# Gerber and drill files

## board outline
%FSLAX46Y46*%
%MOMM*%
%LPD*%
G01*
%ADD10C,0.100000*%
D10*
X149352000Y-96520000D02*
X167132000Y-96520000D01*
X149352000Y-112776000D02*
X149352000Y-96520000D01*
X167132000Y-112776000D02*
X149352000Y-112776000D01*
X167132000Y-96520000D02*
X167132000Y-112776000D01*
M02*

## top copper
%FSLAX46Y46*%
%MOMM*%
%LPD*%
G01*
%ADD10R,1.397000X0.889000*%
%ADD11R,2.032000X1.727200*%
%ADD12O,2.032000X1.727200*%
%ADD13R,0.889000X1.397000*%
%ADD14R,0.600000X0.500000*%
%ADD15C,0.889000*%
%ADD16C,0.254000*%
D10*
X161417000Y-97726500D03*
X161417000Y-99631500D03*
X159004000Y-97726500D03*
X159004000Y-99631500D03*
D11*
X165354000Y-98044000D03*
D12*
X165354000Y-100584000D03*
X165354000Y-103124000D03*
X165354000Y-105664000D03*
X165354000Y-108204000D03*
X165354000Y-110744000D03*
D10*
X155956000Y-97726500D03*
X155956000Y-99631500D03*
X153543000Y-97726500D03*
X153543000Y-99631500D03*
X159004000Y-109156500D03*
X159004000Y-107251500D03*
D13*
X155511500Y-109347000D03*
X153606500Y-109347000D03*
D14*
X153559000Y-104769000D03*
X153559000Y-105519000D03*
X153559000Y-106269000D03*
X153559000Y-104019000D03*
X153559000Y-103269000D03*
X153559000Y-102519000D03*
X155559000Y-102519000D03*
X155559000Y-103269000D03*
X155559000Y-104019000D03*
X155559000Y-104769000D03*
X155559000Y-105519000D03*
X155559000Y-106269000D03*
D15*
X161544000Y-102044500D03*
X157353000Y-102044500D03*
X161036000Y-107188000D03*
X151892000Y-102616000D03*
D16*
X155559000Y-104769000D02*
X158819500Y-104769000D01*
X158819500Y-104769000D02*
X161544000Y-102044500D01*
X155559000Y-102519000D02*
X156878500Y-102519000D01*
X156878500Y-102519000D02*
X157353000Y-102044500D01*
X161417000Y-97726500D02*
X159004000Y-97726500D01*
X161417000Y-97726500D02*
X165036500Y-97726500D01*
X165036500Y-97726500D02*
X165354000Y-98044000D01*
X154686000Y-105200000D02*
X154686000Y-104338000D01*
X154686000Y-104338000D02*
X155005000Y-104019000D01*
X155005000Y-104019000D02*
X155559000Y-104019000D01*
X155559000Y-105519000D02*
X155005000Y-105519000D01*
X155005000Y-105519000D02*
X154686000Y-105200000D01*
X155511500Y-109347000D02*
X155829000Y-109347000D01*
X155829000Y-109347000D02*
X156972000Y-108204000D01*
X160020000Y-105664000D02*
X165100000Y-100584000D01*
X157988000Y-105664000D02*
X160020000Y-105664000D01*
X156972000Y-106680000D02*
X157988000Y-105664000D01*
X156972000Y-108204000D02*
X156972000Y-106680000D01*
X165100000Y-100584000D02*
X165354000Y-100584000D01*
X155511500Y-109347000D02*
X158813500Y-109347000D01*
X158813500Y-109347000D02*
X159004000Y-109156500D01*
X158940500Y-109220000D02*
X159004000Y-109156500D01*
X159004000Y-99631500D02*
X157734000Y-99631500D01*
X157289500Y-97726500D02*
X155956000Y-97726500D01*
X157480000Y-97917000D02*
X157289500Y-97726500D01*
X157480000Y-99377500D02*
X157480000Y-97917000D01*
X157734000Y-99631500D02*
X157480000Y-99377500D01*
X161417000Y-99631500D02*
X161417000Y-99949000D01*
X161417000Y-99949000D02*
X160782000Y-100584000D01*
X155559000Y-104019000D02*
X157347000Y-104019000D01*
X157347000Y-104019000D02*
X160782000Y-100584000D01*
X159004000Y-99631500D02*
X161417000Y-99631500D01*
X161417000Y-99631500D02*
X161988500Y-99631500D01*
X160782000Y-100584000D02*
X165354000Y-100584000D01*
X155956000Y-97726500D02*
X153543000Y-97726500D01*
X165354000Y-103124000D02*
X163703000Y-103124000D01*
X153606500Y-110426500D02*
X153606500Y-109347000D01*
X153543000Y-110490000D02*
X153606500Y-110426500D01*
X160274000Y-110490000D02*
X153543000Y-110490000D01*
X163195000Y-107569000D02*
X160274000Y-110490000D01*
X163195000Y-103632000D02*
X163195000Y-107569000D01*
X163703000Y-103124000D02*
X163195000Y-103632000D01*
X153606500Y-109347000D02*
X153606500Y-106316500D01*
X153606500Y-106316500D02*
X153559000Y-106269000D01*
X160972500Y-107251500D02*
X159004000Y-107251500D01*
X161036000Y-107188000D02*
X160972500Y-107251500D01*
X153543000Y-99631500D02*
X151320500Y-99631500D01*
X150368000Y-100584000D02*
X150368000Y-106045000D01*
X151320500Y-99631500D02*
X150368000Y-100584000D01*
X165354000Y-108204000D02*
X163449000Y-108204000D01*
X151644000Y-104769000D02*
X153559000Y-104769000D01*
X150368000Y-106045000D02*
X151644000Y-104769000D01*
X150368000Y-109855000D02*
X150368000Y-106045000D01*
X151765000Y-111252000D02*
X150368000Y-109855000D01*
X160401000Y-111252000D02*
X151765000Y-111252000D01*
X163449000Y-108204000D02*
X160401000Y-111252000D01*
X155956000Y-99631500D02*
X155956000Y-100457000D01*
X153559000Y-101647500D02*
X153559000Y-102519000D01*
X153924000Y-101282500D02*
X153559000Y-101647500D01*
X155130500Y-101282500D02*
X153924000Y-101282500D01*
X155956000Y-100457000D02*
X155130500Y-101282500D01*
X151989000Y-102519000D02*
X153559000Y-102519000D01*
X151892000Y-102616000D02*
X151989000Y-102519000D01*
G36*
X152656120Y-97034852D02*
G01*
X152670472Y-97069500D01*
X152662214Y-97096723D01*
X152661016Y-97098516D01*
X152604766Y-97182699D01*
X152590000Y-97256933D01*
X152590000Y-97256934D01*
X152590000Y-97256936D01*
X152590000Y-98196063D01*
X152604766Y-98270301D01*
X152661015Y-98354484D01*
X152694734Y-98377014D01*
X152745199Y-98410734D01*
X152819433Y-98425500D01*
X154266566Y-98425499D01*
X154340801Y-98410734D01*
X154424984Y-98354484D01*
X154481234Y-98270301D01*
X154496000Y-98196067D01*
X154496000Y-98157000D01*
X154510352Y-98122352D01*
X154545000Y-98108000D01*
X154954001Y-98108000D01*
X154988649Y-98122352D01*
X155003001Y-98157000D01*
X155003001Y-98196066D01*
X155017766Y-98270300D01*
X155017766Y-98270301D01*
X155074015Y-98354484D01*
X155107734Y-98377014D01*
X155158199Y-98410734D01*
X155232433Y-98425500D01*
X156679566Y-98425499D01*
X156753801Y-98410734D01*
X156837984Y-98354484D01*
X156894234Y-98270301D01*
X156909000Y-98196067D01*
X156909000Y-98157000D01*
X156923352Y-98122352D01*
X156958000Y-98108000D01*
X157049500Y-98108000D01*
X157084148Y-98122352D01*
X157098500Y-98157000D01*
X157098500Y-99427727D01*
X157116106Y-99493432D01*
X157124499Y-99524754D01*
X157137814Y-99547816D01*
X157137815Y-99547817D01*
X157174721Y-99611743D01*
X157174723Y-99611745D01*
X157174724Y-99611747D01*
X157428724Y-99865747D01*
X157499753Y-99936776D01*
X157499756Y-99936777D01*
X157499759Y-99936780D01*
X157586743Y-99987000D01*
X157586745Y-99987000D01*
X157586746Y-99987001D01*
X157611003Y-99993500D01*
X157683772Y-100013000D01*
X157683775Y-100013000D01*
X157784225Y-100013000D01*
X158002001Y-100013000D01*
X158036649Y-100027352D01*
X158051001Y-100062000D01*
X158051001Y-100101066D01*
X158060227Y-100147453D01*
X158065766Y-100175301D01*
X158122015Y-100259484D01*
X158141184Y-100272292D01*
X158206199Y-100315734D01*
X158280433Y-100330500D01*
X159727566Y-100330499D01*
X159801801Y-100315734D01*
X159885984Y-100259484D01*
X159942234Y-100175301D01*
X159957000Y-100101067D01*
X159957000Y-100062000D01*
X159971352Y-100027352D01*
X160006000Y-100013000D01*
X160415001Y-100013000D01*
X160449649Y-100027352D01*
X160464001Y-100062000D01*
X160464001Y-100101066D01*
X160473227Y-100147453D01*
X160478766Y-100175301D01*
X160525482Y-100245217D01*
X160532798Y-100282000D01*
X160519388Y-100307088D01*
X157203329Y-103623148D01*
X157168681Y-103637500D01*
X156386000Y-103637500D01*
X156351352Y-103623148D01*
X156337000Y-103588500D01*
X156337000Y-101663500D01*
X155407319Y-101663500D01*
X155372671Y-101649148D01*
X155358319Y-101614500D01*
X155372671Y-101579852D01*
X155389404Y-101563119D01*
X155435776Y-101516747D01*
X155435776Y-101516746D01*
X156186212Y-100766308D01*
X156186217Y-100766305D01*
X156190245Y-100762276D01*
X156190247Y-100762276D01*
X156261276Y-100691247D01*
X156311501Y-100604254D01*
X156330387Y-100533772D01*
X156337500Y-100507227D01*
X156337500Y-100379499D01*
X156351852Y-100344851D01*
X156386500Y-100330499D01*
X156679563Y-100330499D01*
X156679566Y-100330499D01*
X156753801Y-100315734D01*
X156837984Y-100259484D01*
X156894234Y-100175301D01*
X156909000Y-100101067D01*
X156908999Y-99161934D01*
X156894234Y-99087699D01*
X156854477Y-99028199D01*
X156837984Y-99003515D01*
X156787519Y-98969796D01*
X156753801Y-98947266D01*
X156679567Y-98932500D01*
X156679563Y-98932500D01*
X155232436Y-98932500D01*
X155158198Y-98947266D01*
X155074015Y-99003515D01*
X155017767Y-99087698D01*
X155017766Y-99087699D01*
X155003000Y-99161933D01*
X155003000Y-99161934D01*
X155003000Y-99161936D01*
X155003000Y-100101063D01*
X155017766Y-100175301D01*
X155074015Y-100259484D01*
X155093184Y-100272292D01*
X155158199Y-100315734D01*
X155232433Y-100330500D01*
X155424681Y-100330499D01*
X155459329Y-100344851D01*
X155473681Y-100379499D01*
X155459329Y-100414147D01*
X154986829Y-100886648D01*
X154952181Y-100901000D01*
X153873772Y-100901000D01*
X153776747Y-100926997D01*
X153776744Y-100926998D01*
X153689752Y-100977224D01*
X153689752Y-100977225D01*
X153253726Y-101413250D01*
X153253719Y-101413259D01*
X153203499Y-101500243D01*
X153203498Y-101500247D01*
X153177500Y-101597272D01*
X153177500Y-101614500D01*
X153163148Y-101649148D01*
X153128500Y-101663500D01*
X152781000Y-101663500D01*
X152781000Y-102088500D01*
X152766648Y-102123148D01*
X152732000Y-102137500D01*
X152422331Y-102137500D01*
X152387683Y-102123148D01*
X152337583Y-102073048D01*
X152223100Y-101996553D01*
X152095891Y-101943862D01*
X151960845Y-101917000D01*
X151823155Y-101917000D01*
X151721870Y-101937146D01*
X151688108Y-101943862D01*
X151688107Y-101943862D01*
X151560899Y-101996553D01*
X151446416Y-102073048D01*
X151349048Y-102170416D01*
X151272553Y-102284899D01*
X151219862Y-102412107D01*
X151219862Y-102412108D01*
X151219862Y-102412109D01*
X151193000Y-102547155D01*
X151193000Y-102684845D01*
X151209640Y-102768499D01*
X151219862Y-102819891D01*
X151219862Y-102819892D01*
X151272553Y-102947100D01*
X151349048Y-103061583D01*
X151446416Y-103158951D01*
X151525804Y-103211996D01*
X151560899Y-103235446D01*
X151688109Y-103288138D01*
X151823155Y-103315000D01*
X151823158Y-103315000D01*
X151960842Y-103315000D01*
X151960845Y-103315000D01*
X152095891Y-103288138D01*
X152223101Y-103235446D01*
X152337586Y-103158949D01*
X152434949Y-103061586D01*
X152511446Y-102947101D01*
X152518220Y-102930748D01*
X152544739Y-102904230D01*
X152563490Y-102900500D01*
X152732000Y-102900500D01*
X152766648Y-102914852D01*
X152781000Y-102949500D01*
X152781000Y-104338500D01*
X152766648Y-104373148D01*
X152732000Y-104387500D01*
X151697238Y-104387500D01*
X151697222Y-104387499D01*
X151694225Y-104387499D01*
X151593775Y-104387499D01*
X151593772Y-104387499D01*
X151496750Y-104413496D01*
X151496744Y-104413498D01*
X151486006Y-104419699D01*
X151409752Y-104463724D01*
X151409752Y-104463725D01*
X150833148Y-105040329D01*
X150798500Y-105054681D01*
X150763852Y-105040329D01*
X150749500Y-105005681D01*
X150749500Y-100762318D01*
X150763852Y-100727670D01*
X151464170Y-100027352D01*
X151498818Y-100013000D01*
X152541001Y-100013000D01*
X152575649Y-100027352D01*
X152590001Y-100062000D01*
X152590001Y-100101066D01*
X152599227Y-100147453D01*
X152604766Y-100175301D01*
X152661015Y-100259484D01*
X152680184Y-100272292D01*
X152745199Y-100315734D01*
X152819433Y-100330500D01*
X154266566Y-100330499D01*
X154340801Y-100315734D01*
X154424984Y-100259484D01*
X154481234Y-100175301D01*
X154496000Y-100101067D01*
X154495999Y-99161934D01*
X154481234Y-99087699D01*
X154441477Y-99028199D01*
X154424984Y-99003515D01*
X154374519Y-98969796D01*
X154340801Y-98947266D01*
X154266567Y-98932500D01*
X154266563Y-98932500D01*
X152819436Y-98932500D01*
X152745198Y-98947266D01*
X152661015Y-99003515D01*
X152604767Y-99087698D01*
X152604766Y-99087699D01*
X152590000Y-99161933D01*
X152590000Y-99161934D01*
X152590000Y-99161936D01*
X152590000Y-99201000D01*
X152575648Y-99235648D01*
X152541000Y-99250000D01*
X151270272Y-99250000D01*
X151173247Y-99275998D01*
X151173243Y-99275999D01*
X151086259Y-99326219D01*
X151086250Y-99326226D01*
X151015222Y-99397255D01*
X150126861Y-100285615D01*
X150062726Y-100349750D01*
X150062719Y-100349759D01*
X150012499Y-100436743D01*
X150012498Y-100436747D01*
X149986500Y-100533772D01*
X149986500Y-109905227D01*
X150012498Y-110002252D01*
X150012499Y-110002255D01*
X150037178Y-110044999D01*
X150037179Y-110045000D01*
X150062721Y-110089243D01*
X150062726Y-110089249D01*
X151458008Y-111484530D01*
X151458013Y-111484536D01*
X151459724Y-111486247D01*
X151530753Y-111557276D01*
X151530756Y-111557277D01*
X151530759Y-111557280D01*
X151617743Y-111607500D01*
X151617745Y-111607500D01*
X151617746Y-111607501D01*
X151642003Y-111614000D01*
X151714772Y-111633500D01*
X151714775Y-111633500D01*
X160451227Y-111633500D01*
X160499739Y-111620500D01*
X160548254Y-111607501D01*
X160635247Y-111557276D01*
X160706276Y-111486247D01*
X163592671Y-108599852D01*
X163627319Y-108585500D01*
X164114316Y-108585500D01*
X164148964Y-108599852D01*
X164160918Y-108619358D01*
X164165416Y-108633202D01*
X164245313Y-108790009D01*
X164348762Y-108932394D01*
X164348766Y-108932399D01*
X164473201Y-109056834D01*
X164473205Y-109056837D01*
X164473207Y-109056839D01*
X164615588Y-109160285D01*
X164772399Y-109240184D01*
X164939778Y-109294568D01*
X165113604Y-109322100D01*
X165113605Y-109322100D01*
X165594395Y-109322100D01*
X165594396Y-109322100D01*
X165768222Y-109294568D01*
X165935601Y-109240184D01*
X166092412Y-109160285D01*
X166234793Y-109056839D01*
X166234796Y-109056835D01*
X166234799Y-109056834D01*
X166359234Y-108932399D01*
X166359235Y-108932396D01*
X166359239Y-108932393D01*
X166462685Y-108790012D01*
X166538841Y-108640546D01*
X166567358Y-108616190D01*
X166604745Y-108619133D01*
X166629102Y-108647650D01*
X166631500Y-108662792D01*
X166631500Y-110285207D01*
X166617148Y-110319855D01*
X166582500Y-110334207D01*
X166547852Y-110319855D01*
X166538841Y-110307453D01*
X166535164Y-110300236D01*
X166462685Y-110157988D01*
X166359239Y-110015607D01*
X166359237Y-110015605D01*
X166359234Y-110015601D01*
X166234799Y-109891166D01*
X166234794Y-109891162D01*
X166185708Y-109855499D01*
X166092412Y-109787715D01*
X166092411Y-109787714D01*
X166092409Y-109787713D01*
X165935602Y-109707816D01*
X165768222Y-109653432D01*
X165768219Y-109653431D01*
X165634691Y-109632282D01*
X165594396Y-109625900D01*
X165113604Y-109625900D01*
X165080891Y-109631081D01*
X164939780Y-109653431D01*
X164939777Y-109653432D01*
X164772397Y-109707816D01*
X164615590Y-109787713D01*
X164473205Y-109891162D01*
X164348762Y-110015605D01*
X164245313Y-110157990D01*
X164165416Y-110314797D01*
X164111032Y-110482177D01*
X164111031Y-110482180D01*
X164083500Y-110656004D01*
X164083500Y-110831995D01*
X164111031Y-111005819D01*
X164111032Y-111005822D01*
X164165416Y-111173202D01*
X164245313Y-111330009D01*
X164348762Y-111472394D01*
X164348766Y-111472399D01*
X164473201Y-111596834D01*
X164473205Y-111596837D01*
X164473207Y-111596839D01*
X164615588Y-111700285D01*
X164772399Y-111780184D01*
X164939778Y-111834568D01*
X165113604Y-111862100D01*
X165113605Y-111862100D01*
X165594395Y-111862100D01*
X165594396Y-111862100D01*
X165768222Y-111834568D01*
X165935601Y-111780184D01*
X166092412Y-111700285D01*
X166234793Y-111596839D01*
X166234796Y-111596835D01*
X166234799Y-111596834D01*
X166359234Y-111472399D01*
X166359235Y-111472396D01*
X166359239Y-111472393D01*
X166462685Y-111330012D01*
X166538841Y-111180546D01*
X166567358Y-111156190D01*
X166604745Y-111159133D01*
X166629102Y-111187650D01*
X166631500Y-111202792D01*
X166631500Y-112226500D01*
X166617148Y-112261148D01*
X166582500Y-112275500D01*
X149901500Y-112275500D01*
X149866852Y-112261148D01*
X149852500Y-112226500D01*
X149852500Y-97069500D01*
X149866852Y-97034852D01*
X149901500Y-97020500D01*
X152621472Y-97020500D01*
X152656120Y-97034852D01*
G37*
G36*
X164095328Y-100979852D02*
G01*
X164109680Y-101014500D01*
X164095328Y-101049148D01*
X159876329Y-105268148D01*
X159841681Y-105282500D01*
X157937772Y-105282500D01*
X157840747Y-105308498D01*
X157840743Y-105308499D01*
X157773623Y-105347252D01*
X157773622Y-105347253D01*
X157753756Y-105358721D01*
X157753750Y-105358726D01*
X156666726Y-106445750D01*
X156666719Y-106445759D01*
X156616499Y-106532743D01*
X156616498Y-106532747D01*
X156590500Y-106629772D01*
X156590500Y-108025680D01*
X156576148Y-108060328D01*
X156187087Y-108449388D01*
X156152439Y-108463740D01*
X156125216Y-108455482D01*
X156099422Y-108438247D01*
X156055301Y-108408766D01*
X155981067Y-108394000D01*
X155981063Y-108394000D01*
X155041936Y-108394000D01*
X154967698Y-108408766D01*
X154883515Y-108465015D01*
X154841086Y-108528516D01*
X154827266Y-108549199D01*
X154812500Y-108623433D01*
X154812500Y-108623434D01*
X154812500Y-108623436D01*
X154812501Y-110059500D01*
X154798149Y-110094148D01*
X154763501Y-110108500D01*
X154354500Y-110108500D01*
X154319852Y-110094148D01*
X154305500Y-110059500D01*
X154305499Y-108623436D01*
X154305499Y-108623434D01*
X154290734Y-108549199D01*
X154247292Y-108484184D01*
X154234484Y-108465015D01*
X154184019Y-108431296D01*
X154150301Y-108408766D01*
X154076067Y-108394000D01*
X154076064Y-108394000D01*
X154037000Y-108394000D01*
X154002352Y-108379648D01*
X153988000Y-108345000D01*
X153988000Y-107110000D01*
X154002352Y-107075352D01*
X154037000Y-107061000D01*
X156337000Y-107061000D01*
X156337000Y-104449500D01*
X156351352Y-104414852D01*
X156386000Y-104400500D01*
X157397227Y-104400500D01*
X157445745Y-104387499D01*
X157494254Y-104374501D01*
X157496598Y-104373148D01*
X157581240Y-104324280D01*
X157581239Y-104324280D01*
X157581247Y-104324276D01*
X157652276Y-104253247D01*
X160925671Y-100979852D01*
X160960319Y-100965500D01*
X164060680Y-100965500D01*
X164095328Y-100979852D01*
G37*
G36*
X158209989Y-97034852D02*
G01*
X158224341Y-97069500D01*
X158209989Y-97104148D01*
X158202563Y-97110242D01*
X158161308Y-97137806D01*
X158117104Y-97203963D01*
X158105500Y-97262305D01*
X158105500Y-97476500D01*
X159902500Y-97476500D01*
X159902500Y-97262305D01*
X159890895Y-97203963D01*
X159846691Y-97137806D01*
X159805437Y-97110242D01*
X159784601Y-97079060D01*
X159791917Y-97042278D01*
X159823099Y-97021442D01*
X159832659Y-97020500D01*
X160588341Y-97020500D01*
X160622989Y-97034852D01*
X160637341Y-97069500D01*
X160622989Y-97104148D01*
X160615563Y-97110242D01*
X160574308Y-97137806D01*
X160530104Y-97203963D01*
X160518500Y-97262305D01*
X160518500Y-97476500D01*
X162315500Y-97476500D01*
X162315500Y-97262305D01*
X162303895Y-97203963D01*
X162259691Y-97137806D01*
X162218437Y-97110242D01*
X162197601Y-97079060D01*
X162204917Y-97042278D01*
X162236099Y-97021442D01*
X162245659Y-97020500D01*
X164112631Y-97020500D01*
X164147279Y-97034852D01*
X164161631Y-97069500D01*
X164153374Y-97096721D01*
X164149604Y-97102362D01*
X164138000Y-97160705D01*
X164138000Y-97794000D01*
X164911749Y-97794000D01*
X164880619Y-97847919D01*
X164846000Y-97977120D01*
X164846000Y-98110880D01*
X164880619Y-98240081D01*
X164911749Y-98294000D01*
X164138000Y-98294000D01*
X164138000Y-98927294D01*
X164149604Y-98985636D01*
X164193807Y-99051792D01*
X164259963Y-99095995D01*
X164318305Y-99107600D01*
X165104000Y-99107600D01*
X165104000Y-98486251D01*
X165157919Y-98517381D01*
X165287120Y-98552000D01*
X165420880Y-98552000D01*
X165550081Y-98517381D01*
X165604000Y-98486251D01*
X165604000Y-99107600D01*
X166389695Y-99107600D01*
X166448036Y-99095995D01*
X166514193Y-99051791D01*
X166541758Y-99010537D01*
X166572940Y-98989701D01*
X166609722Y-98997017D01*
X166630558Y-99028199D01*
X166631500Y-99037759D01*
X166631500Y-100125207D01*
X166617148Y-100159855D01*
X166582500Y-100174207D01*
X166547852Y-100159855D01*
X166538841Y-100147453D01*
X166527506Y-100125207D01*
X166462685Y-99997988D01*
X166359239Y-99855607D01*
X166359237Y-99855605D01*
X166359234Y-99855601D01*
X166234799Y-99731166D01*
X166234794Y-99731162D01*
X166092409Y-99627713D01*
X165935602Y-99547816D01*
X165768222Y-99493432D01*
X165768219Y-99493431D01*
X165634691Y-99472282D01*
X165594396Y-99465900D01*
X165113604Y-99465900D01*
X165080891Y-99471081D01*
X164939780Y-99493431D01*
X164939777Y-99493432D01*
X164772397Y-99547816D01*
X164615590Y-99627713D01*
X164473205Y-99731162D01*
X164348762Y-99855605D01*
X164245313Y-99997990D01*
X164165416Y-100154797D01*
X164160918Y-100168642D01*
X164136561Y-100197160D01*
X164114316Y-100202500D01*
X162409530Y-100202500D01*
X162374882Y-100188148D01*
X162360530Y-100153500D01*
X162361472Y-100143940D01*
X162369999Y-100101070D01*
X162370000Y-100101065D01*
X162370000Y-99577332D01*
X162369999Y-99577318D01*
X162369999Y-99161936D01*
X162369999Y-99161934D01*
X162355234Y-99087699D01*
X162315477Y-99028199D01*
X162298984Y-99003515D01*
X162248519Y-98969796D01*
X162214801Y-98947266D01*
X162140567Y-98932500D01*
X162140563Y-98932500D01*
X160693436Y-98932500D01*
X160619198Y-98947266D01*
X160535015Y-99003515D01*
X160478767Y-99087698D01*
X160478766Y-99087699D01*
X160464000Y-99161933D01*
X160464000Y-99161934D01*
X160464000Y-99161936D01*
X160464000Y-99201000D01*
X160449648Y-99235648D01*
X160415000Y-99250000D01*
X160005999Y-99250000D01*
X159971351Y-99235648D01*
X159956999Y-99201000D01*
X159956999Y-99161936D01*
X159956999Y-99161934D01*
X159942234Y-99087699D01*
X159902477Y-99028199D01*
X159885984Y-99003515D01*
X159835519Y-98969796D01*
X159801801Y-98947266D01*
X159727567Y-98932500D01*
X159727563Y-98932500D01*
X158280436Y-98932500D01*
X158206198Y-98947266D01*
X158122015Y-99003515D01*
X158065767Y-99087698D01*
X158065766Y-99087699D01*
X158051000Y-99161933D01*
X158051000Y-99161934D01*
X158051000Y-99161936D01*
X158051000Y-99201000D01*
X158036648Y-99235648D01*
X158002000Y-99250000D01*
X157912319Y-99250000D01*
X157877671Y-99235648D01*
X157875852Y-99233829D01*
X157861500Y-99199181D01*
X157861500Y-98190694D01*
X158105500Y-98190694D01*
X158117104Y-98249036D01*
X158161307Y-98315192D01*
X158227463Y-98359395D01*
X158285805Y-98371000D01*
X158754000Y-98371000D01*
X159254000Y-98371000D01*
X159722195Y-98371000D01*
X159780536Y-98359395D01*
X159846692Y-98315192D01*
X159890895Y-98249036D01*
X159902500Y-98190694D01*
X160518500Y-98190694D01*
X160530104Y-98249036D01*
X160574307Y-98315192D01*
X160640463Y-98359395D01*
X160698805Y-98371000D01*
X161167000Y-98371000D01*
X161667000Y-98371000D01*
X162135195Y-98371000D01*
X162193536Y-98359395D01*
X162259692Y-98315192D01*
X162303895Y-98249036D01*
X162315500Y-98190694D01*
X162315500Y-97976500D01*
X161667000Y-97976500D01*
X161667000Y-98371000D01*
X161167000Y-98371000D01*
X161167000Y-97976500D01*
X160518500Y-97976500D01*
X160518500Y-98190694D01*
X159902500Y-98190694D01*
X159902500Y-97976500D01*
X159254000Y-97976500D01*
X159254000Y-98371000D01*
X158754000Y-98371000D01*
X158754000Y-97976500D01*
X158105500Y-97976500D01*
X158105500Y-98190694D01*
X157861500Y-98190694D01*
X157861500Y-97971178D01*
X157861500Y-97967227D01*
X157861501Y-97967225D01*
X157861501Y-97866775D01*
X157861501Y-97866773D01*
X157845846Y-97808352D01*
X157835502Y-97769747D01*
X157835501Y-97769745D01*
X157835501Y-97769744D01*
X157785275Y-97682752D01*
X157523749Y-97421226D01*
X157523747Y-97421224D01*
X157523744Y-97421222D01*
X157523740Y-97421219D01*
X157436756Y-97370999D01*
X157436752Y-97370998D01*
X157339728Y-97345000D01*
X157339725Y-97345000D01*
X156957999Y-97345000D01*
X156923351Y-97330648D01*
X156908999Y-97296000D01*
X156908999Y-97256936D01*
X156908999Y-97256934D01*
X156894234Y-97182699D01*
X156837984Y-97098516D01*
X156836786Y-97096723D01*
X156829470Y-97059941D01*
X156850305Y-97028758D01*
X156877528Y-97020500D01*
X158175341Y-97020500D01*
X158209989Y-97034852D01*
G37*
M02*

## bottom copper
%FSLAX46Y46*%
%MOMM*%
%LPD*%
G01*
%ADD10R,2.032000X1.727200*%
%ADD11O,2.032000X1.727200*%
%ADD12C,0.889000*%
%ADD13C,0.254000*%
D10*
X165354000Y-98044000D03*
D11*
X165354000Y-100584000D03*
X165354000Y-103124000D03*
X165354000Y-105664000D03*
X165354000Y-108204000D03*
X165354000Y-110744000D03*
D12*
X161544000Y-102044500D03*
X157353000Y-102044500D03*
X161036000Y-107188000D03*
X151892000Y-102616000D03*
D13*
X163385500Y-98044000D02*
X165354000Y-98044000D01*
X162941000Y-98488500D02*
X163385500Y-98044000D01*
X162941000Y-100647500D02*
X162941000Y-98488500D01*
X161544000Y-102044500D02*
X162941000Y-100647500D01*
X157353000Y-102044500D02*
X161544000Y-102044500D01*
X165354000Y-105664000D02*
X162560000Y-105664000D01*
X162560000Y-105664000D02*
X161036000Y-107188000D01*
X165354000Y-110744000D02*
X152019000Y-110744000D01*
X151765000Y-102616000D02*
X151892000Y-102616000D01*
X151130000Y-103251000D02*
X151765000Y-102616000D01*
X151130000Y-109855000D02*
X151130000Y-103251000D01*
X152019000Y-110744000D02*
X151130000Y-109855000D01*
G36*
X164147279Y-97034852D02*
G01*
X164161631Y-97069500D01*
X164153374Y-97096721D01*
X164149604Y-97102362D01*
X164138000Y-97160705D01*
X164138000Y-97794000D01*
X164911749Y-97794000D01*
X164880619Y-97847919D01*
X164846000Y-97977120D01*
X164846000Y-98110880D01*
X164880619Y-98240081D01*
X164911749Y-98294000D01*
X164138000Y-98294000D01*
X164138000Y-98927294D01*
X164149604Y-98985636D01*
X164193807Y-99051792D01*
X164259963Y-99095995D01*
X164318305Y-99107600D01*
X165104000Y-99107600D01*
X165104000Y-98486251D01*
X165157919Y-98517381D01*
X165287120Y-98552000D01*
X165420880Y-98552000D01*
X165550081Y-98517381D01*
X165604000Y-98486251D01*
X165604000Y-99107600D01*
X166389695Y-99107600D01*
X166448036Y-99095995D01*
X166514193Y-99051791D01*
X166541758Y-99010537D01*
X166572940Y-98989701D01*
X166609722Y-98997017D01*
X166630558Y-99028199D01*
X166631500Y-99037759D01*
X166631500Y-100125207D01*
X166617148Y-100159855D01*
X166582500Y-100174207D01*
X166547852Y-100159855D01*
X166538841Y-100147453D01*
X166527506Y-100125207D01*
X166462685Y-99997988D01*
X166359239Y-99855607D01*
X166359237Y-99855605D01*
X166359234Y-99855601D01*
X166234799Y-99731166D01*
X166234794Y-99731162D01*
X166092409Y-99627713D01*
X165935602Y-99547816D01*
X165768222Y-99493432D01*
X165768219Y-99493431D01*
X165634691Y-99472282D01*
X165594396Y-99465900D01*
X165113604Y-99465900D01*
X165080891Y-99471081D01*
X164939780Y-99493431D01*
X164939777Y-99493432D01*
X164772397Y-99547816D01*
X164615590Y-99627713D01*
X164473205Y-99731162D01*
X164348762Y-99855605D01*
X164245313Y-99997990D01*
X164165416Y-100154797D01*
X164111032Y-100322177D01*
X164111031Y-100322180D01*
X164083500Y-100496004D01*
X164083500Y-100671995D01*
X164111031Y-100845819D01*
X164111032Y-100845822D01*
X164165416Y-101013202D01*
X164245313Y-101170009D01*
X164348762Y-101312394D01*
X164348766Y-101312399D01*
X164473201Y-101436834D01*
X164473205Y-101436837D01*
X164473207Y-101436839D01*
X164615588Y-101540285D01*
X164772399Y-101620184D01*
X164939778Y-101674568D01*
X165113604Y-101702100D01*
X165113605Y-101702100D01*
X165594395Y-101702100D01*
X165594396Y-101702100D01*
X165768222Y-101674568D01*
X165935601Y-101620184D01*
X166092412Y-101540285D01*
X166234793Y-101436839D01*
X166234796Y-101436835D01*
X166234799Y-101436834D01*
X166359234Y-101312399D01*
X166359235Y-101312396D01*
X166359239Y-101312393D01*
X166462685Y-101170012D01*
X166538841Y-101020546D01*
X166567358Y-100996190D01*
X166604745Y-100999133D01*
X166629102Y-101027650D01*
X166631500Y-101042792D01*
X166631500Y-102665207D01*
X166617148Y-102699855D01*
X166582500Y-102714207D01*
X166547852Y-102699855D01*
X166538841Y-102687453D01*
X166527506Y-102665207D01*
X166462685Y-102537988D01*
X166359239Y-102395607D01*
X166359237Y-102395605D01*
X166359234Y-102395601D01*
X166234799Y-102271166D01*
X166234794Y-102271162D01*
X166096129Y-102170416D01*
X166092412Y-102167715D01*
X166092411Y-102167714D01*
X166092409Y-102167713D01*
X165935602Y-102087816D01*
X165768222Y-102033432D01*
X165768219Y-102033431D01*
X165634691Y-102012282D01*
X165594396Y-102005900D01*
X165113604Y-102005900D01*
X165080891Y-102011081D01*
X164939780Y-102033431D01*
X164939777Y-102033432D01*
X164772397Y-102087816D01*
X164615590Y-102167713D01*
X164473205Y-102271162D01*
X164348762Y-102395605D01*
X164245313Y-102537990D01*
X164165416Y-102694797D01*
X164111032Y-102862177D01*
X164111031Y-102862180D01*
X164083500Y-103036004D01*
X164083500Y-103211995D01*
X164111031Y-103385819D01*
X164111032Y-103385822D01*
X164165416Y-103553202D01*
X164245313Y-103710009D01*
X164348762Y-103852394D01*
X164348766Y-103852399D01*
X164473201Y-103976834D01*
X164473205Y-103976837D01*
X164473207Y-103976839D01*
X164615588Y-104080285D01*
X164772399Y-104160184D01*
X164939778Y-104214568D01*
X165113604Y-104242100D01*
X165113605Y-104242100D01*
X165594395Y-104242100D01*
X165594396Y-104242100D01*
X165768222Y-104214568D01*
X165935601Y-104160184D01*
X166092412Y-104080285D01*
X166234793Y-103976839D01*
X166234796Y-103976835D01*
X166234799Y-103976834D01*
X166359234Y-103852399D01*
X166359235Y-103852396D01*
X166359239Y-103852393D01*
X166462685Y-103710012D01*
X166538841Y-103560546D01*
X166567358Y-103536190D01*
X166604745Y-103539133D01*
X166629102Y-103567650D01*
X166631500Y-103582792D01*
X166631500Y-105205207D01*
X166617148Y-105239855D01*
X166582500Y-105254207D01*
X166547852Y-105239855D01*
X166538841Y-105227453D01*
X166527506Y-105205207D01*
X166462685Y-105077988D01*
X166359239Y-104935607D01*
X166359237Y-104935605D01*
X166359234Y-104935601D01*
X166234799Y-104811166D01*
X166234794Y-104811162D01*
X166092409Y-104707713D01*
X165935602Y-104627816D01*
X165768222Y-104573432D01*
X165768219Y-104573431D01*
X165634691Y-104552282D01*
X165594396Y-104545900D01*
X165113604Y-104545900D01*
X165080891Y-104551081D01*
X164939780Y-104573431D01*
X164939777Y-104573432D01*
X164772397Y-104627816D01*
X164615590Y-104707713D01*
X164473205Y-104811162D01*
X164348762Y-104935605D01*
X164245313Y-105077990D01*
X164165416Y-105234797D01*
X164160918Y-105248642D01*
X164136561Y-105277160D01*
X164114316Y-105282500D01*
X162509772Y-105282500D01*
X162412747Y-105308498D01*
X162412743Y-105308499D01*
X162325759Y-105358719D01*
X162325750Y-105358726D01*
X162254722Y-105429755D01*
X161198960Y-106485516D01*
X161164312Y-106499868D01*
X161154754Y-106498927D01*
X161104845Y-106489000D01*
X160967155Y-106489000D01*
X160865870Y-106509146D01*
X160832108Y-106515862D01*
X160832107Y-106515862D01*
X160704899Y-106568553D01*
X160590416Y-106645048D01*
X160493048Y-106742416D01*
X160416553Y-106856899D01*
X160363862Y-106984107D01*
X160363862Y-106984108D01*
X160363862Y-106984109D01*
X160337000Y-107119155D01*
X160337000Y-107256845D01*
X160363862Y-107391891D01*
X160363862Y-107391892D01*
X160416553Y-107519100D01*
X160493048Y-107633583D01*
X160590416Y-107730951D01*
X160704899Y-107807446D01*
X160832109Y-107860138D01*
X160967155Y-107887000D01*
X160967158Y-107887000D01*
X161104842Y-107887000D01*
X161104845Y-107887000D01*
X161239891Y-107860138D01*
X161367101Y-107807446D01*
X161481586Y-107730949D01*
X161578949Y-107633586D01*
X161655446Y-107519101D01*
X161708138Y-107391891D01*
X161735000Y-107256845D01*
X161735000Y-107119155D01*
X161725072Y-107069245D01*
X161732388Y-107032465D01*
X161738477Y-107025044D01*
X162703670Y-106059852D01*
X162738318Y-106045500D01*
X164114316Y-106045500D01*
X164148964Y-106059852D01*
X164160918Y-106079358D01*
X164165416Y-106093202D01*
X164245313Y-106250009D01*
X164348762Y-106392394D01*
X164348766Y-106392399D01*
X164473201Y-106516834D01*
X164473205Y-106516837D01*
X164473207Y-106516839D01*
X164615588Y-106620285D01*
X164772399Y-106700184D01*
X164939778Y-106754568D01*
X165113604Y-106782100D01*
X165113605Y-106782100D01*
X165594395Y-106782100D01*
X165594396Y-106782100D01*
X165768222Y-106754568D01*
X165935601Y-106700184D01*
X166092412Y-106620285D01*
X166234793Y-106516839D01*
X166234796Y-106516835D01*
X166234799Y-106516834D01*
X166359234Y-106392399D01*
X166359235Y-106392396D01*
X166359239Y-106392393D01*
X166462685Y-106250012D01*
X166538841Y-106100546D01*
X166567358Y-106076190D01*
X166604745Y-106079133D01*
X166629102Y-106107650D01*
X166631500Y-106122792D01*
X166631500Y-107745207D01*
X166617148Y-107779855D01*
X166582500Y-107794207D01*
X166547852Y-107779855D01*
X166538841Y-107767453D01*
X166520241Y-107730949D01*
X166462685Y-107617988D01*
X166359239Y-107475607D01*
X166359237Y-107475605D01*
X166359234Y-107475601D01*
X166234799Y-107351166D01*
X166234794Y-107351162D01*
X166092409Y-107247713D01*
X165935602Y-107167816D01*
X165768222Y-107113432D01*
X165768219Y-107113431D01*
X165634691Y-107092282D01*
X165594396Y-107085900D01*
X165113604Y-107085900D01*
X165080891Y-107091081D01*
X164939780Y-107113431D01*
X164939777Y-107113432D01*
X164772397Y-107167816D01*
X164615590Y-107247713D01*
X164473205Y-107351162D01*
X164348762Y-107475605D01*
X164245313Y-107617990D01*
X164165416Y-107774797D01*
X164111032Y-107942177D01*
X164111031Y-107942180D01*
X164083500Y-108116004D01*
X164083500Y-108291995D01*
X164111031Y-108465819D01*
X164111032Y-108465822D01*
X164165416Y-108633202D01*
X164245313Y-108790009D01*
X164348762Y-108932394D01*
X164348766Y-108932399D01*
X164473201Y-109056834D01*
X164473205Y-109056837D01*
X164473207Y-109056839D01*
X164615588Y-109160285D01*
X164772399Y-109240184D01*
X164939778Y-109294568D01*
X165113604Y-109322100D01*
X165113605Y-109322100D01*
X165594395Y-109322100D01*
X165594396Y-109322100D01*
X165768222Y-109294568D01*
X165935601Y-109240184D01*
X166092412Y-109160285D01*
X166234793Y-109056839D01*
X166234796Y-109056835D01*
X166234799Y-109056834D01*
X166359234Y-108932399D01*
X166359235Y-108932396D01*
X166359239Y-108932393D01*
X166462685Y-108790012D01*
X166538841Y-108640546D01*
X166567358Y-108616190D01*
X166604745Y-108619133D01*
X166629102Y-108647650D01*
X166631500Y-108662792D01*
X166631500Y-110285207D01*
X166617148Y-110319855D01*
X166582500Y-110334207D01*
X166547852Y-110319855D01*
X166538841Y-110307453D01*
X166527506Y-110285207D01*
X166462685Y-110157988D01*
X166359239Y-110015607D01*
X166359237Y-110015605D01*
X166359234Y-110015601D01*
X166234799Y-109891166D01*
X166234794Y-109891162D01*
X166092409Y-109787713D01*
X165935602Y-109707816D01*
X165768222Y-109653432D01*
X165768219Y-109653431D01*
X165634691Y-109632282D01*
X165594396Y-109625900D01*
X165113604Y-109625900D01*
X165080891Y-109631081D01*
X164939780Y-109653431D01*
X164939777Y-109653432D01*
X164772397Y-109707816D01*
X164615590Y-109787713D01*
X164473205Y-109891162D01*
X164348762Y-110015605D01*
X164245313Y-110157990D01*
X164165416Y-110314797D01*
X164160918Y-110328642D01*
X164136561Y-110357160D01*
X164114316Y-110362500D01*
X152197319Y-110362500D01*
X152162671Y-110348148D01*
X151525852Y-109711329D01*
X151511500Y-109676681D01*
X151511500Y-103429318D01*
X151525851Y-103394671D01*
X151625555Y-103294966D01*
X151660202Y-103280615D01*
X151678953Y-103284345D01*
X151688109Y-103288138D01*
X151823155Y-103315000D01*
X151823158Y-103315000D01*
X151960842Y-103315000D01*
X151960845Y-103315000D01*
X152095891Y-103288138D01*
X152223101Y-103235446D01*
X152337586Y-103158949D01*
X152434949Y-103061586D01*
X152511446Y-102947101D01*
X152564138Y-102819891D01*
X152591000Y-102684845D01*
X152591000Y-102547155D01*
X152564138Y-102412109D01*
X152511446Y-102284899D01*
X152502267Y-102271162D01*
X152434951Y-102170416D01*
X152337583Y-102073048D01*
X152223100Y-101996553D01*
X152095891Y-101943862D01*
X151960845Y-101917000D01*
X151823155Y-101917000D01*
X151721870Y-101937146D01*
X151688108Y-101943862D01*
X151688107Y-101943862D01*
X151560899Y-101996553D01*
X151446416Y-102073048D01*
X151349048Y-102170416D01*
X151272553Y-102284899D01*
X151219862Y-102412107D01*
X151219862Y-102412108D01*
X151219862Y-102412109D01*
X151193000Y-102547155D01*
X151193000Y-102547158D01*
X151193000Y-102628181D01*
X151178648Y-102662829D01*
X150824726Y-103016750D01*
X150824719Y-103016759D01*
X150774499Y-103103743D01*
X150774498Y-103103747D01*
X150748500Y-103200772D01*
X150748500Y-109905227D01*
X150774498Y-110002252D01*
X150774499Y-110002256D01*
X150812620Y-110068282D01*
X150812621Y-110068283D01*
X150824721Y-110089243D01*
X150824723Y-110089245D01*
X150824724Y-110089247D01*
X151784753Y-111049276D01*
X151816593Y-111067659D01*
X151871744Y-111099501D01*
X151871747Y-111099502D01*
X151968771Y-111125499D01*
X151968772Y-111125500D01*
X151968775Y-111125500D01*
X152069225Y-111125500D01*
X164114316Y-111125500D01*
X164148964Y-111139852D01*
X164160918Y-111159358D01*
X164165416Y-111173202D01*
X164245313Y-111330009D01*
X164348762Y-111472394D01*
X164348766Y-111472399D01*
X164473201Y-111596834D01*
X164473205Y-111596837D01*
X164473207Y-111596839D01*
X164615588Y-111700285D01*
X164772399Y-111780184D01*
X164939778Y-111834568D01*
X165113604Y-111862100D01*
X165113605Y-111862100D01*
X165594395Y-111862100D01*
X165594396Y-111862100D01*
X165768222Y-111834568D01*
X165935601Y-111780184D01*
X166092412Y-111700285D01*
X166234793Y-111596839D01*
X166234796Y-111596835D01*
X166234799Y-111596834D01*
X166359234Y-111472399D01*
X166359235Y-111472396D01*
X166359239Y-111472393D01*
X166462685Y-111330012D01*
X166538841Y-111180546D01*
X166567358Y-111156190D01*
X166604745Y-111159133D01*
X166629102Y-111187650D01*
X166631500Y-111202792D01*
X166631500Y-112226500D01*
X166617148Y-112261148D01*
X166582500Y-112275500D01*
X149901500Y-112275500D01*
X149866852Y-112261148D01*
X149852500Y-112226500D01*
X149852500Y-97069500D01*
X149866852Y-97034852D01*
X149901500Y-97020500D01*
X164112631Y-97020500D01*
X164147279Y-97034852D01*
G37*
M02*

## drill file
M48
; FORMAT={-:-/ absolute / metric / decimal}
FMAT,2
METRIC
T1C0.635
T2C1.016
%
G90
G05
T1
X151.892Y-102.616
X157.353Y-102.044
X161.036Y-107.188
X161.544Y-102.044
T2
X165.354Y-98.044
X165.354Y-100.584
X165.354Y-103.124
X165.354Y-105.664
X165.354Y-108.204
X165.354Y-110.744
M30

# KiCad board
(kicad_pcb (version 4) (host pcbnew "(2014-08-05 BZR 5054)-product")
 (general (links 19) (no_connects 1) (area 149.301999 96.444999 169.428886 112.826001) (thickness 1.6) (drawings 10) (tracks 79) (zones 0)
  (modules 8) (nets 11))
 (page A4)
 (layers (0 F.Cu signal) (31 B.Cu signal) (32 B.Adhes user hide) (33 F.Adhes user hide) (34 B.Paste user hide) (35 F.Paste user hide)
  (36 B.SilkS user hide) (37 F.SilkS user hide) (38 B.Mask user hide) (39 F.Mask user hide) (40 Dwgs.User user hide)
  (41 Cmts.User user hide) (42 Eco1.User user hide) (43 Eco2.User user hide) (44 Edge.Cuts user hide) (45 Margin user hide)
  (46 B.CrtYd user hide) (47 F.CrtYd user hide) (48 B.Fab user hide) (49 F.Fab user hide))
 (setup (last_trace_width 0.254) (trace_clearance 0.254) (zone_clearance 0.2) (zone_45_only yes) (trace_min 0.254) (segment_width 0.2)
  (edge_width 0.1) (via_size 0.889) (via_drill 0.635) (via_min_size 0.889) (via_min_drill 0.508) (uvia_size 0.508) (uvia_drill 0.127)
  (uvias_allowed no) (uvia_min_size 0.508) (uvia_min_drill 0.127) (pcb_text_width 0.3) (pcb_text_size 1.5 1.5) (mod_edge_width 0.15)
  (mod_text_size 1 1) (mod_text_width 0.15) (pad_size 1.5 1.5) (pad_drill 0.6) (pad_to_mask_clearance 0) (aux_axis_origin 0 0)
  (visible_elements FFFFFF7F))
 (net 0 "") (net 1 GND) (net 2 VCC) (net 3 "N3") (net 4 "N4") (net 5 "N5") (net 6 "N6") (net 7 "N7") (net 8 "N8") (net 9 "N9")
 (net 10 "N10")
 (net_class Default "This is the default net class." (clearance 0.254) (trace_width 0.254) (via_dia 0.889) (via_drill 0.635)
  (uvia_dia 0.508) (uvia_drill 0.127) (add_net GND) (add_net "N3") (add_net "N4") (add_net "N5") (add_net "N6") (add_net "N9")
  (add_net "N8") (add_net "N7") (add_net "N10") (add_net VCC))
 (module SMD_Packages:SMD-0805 (layer F.Cu) (at 161.417 98.679 270)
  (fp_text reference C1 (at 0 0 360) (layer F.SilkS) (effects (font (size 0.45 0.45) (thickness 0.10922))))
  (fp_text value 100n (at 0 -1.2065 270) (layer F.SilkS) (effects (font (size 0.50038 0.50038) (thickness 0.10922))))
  (pad 1 smd rect (at -0.9525 0 270) (size 0.889 1.397) (layers F.Cu F.Paste F.Mask) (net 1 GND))
  (pad 2 smd rect (at 0.9525 0 270) (size 0.889 1.397) (layers F.Cu F.Paste F.Mask) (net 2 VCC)))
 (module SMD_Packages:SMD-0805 (layer F.Cu) (at 159.004 98.679 270)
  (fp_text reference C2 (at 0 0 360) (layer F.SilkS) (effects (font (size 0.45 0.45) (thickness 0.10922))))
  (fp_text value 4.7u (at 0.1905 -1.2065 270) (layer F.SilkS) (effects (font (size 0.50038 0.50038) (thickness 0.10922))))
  (pad 1 smd rect (at -0.9525 0 270) (size 0.889 1.397) (layers F.Cu F.Paste F.Mask) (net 1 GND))
  (pad 2 smd rect (at 0.9525 0 270) (size 0.889 1.397) (layers F.Cu F.Paste F.Mask) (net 2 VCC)))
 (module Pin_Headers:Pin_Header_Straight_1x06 (layer F.Cu) (at 165.354 104.394 270)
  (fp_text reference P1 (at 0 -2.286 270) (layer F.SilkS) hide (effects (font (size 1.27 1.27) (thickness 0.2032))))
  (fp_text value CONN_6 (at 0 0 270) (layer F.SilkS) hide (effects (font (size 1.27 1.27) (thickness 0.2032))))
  (pad 1 thru_hole rect (at -6.35 0 270) (size 1.7272 2.032) (drill 1.016) (layers *.Cu *.Mask F.SilkS) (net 1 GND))
  (pad 2 thru_hole oval (at -3.81 0 270) (size 1.7272 2.032) (drill 1.016) (layers *.Cu *.Mask F.SilkS) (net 2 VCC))
  (pad 3 thru_hole oval (at -1.27 0 270) (size 1.7272 2.032) (drill 1.016) (layers *.Cu *.Mask F.SilkS) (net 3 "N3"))
  (pad 4 thru_hole oval (at 1.27 0 270) (size 1.7272 2.032) (drill 1.016) (layers *.Cu *.Mask F.SilkS) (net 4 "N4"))
  (pad 5 thru_hole oval (at 3.81 0 270) (size 1.7272 2.032) (drill 1.016) (layers *.Cu *.Mask F.SilkS) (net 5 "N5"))
  (pad 6 thru_hole oval (at 6.35 0 270) (size 1.7272 2.032) (drill 1.016) (layers *.Cu *.Mask F.SilkS) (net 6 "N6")))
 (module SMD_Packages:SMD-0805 (layer F.Cu) (at 155.956 98.679 270)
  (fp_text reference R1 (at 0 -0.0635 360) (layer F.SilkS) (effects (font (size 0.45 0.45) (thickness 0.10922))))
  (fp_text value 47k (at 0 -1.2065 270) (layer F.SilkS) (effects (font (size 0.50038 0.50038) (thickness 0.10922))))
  (pad 1 smd rect (at -0.9525 0 270) (size 0.889 1.397) (layers F.Cu F.Paste F.Mask) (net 2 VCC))
  (pad 2 smd rect (at 0.9525 0 270) (size 0.889 1.397) (layers F.Cu F.Paste F.Mask) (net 6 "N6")))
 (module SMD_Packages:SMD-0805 (layer F.Cu) (at 153.543 98.679 270)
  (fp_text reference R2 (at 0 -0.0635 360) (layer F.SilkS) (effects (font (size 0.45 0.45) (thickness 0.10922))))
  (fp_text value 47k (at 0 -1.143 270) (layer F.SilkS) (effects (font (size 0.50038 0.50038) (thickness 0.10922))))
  (pad 1 smd rect (at -0.9525 0 270) (size 0.889 1.397) (layers F.Cu F.Paste F.Mask) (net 2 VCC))
  (pad 2 smd rect (at 0.9525 0 270) (size 0.889 1.397) (layers F.Cu F.Paste F.Mask) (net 5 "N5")))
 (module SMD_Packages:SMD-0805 (layer F.Cu) (at 159.004 108.204 90)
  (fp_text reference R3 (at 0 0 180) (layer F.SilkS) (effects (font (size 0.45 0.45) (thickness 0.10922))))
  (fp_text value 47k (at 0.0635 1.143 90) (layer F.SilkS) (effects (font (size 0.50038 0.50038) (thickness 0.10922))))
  (pad 1 smd rect (at -0.9525 0 90) (size 0.889 1.397) (layers F.Cu F.Paste F.Mask) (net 2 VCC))
  (pad 2 smd rect (at 0.9525 0 90) (size 0.889 1.397) (layers F.Cu F.Paste F.Mask) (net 4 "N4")))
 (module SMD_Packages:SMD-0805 (layer F.Cu) (at 154.559 109.347 180)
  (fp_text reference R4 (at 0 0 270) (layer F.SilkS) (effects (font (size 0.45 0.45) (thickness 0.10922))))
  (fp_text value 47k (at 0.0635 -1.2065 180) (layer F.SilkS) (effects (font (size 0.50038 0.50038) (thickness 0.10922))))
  (pad 1 smd rect (at -0.9525 0 180) (size 0.889 1.397) (layers F.Cu F.Paste F.Mask) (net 2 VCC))
  (pad 2 smd rect (at 0.9525 0 180) (size 0.889 1.397) (layers F.Cu F.Paste F.Mask) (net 3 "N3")))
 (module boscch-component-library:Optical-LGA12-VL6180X (layer F.Cu) (at 154.559 104.394)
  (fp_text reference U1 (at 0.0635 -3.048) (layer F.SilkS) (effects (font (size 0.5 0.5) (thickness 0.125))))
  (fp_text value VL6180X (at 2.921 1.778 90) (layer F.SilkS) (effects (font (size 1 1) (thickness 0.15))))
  (pad 4 smd rect (at -1 0.375) (size 0.6 0.5) (layers F.Cu F.Paste F.Mask) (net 5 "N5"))
  (pad 5 smd rect (at -1 1.125) (size 0.6 0.5) (layers F.Cu F.Paste F.Mask))
  (pad 6 smd rect (at -1 1.875) (size 0.6 0.5) (layers F.Cu F.Paste F.Mask) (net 3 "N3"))
  (pad 3 smd rect (at -1 -0.375) (size 0.6 0.5) (layers F.Cu F.Paste F.Mask) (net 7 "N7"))
  (pad 2 smd rect (at -1 -1.125) (size 0.6 0.5) (layers F.Cu F.Paste F.Mask) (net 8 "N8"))
  (pad 1 smd rect (at -1 -1.875) (size 0.6 0.5) (layers F.Cu F.Paste F.Mask) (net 6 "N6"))
  (pad 12 smd rect (at 1 -1.875) (size 0.6 0.5) (layers F.Cu F.Paste F.Mask) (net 1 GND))
  (pad 11 smd rect (at 1 -1.125) (size 0.6 0.5) (layers F.Cu F.Paste F.Mask) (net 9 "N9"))
  (pad 10 smd rect (at 1 -0.375) (size 0.6 0.5) (layers F.Cu F.Paste F.Mask) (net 2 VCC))
  (pad 9 smd rect (at 1 0.375) (size 0.6 0.5) (layers F.Cu F.Paste F.Mask) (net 1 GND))
  (pad 8 smd rect (at 1 1.125) (size 0.6 0.5) (layers F.Cu F.Paste F.Mask) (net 2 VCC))
  (pad 7 smd rect (at 1 1.875) (size 0.6 0.5) (layers F.Cu F.Paste F.Mask) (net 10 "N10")))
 (gr_line (start 149.352 96.52) (end 167.132 96.52) (angle 90) (layer Edge.Cuts) (width 0.1))
 (gr_line (start 149.352 112.776) (end 149.352 96.52) (angle 90) (layer Edge.Cuts) (width 0.1))
 (gr_line (start 167.132 112.776) (end 149.352 112.776) (angle 90) (layer Edge.Cuts) (width 0.1))
 (gr_line (start 167.132 96.52) (end 167.132 112.776) (angle 90) (layer Edge.Cuts) (width 0.1))
 (segment (start 155.559 104.769) (end 158.8195 104.769) (width 0.254) (layer F.Cu) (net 1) (status 10))
 (via (at 161.544 102.0445) (size 0.889) (layers F.Cu B.Cu) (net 1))
 (segment (start 158.8195 104.769) (end 161.544 102.0445) (width 0.254) (layer F.Cu) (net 1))
 (segment (start 155.559 102.519) (end 156.8785 102.519) (width 0.254) (layer F.Cu) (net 1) (status 10))
 (segment (start 163.3855 98.044) (end 165.354 98.044) (width 0.254) (layer B.Cu) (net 1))
 (segment (start 162.941 98.4885) (end 163.3855 98.044) (width 0.254) (layer B.Cu) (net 1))
 (segment (start 162.941 100.6475) (end 162.941 98.4885) (width 0.254) (layer B.Cu) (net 1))
 (segment (start 161.544 102.0445) (end 162.941 100.6475) (width 0.254) (layer B.Cu) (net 1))
 (segment (start 157.353 102.0445) (end 161.544 102.0445) (width 0.254) (layer B.Cu) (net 1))
 (via (at 157.353 102.0445) (size 0.889) (layers F.Cu B.Cu) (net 1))
 (segment (start 156.8785 102.519) (end 157.353 102.0445) (width 0.254) (layer F.Cu) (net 1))
 (segment (start 161.417 97.7265) (end 159.004 97.7265) (width 0.254) (layer F.Cu) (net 1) (status 20))
 (segment (start 161.417 97.7265) (end 165.0365 97.7265) (width 0.254) (layer F.Cu) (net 1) (status 10))
 (segment (start 165.0365 97.7265) (end 165.354 98.044) (width 0.254) (layer F.Cu) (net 1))
 (segment (start 154.686 105.2) (end 154.686 104.338) (width 0.254) (layer F.Cu) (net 2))
 (segment (start 154.686 104.338) (end 155.005 104.019) (width 0.254) (layer F.Cu) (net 2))
 (segment (start 155.005 104.019) (end 155.559 104.019) (width 0.254) (layer F.Cu) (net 2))
 (segment (start 155.559 105.519) (end 155.005 105.519) (width 0.254) (layer F.Cu) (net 2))
 (segment (start 155.005 105.519) (end 154.686 105.2) (width 0.254) (layer F.Cu) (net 2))
 (segment (start 155.5115 109.347) (end 155.829 109.347) (width 0.254) (layer F.Cu) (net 2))
 (segment (start 155.829 109.347) (end 156.972 108.204) (width 0.254) (layer F.Cu) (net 2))
 (segment (start 160.02 105.664) (end 165.1 100.584) (width 0.254) (layer F.Cu) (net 2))
 (segment (start 157.988 105.664) (end 160.02 105.664) (width 0.254) (layer F.Cu) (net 2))
 (segment (start 156.972 106.68) (end 157.988 105.664) (width 0.254) (layer F.Cu) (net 2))
 (segment (start 156.972 108.204) (end 156.972 106.68) (width 0.254) (layer F.Cu) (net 2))
 (segment (start 165.1 100.584) (end 165.354 100.584) (width 0.254) (layer F.Cu) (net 2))
 (segment (start 155.5115 109.347) (end 158.8135 109.347) (width 0.254) (layer F.Cu) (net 2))
 (segment (start 158.8135 109.347) (end 159.004 109.1565) (width 0.254) (layer F.Cu) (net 2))
 (segment (start 158.9405 109.22) (end 159.004 109.1565) (width 0.254) (layer F.Cu) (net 2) (status 30))
 (segment (start 159.004 99.6315) (end 157.734 99.6315) (width 0.254) (layer F.Cu) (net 2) (status 10))
 (segment (start 157.2895 97.7265) (end 155.956 97.7265) (width 0.254) (layer F.Cu) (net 2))
 (segment (start 157.48 97.917) (end 157.2895 97.7265) (width 0.254) (layer F.Cu) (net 2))
 (segment (start 157.48 99.3775) (end 157.48 97.917) (width 0.254) (layer F.Cu) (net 2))
 (segment (start 157.734 99.6315) (end 157.48 99.3775) (width 0.254) (layer F.Cu) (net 2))
 (segment (start 161.417 99.6315) (end 161.417 99.949) (width 0.254) (layer F.Cu) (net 2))
 (segment (start 161.417 99.949) (end 160.782 100.584) (width 0.254) (layer F.Cu) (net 2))
 (segment (start 155.559 104.019) (end 157.347 104.019) (width 0.254) (layer F.Cu) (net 2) (status 10))
 (segment (start 157.347 104.019) (end 160.782 100.584) (width 0.254) (layer F.Cu) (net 2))
 (segment (start 159.004 99.6315) (end 161.417 99.6315) (width 0.254) (layer F.Cu) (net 2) (status 10))
 (segment (start 161.417 99.6315) (end 161.9885 99.6315) (width 0.254) (layer F.Cu) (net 2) (status 30))
 (segment (start 160.782 100.584) (end 165.354 100.584) (width 0.254) (layer F.Cu) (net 2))
 (segment (start 155.956 97.7265) (end 153.543 97.7265) (width 0.254) (layer F.Cu) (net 2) (status 20))
 (segment (start 165.354 103.124) (end 163.703 103.124) (width 0.254) (layer F.Cu) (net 3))
 (segment (start 153.6065 110.4265) (end 153.6065 109.347) (width 0.254) (layer F.Cu) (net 3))
 (segment (start 153.543 110.49) (end 153.6065 110.4265) (width 0.254) (layer F.Cu) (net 3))
 (segment (start 160.274 110.49) (end 153.543 110.49) (width 0.254) (layer F.Cu) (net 3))
 (segment (start 163.195 107.569) (end 160.274 110.49) (width 0.254) (layer F.Cu) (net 3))
 (segment (start 163.195 103.632) (end 163.195 107.569) (width 0.254) (layer F.Cu) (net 3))
 (segment (start 163.703 103.124) (end 163.195 103.632) (width 0.254) (layer F.Cu) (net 3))
 (segment (start 153.6065 109.347) (end 153.6065 106.3165) (width 0.254) (layer F.Cu) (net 3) (status 20))
 (segment (start 153.6065 106.3165) (end 153.559 106.269) (width 0.254) (layer F.Cu) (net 3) (status 30))
 (segment (start 165.354 105.664) (end 162.56 105.664) (width 0.254) (layer B.Cu) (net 4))
 (segment (start 160.9725 107.2515) (end 159.004 107.2515) (width 0.254) (layer F.Cu) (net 4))
 (segment (start 161.036 107.188) (end 160.9725 107.2515) (width 0.254) (layer F.Cu) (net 4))
 (via (at 161.036 107.188) (size 0.889) (layers F.Cu B.Cu) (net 4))
 (segment (start 162.56 105.664) (end 161.036 107.188) (width 0.254) (layer B.Cu) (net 4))
 (segment (start 153.543 99.6315) (end 151.3205 99.6315) (width 0.254) (layer F.Cu) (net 5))
 (segment (start 150.368 100.584) (end 150.368 106.045) (width 0.254) (layer F.Cu) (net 5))
 (segment (start 151.3205 99.6315) (end 150.368 100.584) (width 0.254) (layer F.Cu) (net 5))
 (segment (start 165.354 108.204) (end 163.449 108.204) (width 0.254) (layer F.Cu) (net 5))
 (segment (start 151.644 104.769) (end 153.559 104.769) (width 0.254) (layer F.Cu) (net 5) (status 20))
 (segment (start 150.368 106.045) (end 151.644 104.769) (width 0.254) (layer F.Cu) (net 5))
 (segment (start 150.368 109.855) (end 150.368 106.045) (width 0.254) (layer F.Cu) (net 5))
 (segment (start 151.765 111.252) (end 150.368 109.855) (width 0.254) (layer F.Cu) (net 5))
 (segment (start 160.401 111.252) (end 151.765 111.252) (width 0.254) (layer F.Cu) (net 5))
 (segment (start 163.449 108.204) (end 160.401 111.252) (width 0.254) (layer F.Cu) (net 5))
 (segment (start 155.956 99.6315) (end 155.956 100.457) (width 0.254) (layer F.Cu) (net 6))
 (segment (start 153.559 101.6475) (end 153.559 102.519) (width 0.254) (layer F.Cu) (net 6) (status 20))
 (segment (start 153.924 101.2825) (end 153.559 101.6475) (width 0.254) (layer F.Cu) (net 6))
 (segment (start 155.1305 101.2825) (end 153.924 101.2825) (width 0.254) (layer F.Cu) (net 6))
 (segment (start 155.956 100.457) (end 155.1305 101.2825) (width 0.254) (layer F.Cu) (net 6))
 (segment (start 165.354 110.744) (end 152.019 110.744) (width 0.254) (layer B.Cu) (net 6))
 (segment (start 151.989 102.519) (end 153.559 102.519) (width 0.254) (layer F.Cu) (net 6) (status 20))
 (segment (start 151.892 102.616) (end 151.989 102.519) (width 0.254) (layer F.Cu) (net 6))
 (via (at 151.892 102.616) (size 0.889) (layers F.Cu B.Cu) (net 6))
 (segment (start 151.765 102.616) (end 151.892 102.616) (width 0.254) (layer B.Cu) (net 6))
 (segment (start 151.13 103.251) (end 151.765 102.616) (width 0.254) (layer B.Cu) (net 6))
 (segment (start 151.13 109.855) (end 151.13 103.251) (width 0.254) (layer B.Cu) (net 6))
 (segment (start 152.019 110.744) (end 151.13 109.855) (width 0.254) (layer B.Cu) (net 6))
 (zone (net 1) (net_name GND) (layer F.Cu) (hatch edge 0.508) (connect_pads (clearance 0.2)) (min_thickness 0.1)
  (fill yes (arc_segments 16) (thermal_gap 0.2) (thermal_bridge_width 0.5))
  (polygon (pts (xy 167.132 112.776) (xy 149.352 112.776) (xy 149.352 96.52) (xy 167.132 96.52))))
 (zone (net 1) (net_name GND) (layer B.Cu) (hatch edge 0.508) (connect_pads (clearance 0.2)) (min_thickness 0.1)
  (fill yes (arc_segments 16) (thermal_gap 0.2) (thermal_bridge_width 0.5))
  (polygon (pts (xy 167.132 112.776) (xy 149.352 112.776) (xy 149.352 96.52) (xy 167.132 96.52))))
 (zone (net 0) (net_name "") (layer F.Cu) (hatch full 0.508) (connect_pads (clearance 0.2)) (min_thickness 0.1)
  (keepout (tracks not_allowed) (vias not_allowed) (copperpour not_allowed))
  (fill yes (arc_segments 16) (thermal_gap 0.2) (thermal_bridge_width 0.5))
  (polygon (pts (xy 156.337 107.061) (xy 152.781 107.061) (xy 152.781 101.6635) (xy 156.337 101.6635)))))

